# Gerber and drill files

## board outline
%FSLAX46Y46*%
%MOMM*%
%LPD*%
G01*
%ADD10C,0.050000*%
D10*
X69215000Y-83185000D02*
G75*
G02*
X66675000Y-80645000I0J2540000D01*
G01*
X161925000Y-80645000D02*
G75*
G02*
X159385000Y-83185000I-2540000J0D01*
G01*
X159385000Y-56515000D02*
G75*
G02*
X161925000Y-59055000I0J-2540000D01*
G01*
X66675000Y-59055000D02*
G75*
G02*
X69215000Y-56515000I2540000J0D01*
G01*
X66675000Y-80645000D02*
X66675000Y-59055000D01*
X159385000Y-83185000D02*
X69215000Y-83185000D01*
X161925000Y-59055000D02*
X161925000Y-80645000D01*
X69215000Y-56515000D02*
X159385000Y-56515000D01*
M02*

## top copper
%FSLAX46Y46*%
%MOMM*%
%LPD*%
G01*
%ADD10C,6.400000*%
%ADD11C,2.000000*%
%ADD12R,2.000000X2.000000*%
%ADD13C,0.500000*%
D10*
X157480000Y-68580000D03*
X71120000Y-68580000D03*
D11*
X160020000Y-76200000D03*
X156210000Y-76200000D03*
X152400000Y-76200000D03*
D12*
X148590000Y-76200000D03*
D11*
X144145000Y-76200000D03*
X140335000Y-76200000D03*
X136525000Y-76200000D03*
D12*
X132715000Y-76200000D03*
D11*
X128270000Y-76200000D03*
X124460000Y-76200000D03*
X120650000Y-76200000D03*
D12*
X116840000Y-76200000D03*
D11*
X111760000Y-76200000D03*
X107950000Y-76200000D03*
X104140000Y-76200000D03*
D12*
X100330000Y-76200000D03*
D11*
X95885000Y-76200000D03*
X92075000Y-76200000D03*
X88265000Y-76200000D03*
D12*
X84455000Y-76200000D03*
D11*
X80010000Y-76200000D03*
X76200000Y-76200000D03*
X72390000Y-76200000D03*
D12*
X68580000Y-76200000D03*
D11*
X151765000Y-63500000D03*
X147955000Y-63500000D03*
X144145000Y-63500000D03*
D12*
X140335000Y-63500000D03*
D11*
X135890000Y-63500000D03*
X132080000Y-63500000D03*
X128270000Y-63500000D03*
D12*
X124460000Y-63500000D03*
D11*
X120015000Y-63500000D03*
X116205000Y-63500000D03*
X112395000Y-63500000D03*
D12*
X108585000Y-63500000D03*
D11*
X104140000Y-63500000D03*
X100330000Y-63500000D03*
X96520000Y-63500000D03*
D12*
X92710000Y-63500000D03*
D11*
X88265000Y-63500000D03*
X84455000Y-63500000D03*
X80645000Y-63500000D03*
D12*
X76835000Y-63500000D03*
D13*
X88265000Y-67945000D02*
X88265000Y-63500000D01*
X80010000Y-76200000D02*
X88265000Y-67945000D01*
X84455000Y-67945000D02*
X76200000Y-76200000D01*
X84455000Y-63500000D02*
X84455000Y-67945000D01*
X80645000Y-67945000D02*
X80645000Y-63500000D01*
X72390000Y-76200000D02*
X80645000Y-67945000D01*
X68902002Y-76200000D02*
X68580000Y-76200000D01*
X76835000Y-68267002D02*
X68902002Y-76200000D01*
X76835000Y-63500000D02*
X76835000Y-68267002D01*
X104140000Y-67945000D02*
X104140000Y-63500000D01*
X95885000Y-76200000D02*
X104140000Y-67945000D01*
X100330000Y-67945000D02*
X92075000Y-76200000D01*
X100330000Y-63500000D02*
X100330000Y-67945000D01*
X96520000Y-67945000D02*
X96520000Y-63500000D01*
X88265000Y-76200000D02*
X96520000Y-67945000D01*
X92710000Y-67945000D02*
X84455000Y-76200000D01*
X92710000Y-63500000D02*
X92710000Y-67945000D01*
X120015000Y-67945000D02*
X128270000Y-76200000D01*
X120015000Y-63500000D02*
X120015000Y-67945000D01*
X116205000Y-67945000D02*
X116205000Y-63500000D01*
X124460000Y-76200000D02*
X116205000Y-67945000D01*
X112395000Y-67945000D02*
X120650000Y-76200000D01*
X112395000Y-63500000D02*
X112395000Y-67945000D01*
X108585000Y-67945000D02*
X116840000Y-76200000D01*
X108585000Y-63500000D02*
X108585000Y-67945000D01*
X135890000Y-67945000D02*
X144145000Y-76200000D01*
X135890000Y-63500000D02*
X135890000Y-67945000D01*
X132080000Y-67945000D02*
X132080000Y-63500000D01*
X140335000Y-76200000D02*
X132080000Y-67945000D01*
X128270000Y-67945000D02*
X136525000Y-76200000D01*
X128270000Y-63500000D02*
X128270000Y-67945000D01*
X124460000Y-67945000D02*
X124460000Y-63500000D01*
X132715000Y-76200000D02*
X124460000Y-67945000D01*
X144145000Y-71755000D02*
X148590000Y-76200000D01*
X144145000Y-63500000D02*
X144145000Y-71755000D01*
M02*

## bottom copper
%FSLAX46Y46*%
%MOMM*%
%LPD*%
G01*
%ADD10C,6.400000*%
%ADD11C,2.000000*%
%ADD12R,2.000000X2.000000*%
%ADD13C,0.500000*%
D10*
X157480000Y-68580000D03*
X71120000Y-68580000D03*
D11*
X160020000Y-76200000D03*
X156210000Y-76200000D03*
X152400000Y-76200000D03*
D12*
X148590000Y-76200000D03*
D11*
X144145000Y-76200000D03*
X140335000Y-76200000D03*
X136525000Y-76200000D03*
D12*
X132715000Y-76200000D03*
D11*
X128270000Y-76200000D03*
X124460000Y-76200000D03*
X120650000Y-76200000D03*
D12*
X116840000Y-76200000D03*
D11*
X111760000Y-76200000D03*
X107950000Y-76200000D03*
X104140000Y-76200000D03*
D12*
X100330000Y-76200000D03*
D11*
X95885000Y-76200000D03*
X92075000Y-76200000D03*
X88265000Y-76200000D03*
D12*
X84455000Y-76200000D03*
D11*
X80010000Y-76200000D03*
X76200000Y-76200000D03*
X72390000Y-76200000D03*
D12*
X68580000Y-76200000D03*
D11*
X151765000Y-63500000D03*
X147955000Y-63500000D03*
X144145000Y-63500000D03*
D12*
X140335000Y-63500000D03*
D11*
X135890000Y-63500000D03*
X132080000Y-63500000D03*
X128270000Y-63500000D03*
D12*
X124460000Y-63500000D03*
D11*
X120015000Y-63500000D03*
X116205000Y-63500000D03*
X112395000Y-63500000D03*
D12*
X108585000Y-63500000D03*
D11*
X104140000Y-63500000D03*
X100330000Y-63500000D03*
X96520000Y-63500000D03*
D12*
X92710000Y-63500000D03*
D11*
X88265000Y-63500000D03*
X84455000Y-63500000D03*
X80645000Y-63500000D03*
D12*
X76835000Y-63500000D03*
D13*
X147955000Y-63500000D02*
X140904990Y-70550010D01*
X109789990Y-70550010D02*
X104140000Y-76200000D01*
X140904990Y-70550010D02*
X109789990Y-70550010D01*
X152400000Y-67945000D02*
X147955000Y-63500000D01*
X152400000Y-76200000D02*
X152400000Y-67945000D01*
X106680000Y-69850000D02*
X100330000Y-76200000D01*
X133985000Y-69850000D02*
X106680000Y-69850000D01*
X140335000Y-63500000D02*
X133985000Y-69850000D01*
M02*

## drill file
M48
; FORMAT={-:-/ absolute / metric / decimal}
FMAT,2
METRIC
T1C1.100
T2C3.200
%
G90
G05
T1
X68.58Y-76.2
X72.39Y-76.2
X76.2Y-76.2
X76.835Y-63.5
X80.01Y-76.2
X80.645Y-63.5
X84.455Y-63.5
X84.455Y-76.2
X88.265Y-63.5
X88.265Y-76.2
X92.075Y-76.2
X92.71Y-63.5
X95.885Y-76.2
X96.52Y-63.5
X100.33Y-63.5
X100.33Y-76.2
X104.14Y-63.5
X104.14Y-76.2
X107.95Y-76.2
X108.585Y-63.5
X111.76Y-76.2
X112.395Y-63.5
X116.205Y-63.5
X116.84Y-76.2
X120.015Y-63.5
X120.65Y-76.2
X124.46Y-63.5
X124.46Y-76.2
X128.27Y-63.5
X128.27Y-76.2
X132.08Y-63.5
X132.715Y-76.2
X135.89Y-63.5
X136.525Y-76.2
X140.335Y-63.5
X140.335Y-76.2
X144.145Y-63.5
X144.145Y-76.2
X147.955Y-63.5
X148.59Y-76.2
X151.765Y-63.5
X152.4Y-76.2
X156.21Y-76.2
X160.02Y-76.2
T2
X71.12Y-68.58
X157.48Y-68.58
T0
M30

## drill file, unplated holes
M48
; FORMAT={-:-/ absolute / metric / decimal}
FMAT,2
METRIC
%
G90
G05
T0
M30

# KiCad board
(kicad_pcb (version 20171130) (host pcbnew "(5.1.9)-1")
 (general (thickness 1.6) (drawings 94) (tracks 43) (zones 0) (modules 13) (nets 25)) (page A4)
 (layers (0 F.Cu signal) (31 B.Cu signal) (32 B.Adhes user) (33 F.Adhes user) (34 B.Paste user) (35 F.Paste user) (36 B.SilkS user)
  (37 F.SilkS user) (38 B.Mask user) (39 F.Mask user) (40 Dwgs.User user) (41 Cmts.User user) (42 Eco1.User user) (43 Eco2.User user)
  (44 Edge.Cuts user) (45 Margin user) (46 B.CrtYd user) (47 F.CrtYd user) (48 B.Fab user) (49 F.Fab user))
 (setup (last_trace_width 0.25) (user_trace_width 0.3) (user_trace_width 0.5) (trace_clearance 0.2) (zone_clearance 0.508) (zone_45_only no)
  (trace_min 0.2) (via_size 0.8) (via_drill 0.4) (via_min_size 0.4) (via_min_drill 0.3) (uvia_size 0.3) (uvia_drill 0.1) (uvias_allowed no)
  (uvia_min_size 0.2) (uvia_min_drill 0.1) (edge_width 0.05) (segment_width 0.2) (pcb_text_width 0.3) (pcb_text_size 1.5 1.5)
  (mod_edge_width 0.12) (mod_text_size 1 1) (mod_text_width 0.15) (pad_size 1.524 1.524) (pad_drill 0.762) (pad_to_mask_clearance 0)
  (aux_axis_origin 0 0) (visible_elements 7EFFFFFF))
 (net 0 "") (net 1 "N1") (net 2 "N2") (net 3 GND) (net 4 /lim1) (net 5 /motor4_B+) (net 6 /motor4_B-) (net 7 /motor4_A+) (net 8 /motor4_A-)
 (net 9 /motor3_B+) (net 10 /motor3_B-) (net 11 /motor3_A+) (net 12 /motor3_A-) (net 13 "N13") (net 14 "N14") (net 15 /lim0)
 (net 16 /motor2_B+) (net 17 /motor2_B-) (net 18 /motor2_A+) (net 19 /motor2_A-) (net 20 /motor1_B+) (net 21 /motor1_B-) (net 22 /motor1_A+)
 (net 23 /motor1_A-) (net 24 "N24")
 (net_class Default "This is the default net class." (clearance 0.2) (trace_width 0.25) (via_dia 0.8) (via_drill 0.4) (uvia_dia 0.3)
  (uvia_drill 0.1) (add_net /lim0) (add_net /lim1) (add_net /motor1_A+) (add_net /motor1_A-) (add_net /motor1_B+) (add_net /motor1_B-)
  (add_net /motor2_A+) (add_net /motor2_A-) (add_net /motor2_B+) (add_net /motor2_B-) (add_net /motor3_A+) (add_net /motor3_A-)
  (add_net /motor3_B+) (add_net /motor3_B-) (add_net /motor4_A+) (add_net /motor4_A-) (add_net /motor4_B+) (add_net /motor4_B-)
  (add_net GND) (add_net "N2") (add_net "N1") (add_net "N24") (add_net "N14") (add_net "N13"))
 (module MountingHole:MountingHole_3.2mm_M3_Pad (layer F.Cu) (at 157.48 68.58)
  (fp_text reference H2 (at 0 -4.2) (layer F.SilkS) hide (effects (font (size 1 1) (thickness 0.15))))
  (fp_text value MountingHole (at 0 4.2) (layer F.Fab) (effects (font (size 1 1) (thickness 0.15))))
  (pad 1 thru_hole circle (at 0 0) (size 6.4 6.4) (drill 3.2) (layers *.Cu *.Mask)))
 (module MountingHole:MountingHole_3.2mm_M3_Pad (layer F.Cu) (at 71.12 68.58)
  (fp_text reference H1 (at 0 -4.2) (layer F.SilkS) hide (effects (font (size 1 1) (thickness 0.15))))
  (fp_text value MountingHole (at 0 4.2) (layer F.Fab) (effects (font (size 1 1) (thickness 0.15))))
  (pad 1 thru_hole circle (at 0 0) (size 6.4 6.4) (drill 3.2) (layers *.Cu *.Mask)))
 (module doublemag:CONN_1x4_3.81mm (layer F.Cu) (at 148.59 76.2)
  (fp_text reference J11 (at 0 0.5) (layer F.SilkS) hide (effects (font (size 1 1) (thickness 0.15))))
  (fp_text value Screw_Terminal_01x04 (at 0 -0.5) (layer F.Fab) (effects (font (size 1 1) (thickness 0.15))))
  (pad 4 thru_hole circle (at 11.43 0 90) (size 2 2) (drill 1.1) (layers *.Cu *.Mask) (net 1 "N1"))
  (pad 3 thru_hole circle (at 7.62 0 90) (size 2 2) (drill 1.1) (layers *.Cu *.Mask) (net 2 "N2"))
  (pad 2 thru_hole circle (at 3.81 0 90) (size 2 2) (drill 1.1) (layers *.Cu *.Mask) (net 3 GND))
  (pad 1 thru_hole rect (at 0 0 90) (size 2 2) (drill 1.1) (layers *.Cu *.Mask) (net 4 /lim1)))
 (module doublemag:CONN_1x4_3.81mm (layer F.Cu) (at 132.715 76.2)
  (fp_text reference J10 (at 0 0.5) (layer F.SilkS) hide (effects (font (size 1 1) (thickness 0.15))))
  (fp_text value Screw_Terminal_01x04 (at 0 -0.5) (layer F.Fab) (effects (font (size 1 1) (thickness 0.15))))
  (pad 4 thru_hole circle (at 11.43 0 90) (size 2 2) (drill 1.1) (layers *.Cu *.Mask) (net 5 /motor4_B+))
  (pad 3 thru_hole circle (at 7.62 0 90) (size 2 2) (drill 1.1) (layers *.Cu *.Mask) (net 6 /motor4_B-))
  (pad 2 thru_hole circle (at 3.81 0 90) (size 2 2) (drill 1.1) (layers *.Cu *.Mask) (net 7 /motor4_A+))
  (pad 1 thru_hole rect (at 0 0 90) (size 2 2) (drill 1.1) (layers *.Cu *.Mask) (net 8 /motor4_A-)))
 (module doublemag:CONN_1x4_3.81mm (layer F.Cu) (at 116.84 76.2)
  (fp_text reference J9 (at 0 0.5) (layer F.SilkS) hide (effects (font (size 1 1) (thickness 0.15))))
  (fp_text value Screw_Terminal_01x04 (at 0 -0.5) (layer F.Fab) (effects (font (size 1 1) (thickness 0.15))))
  (pad 4 thru_hole circle (at 11.43 0 90) (size 2 2) (drill 1.1) (layers *.Cu *.Mask) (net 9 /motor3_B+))
  (pad 3 thru_hole circle (at 7.62 0 90) (size 2 2) (drill 1.1) (layers *.Cu *.Mask) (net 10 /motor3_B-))
  (pad 2 thru_hole circle (at 3.81 0 90) (size 2 2) (drill 1.1) (layers *.Cu *.Mask) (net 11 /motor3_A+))
  (pad 1 thru_hole rect (at 0 0 90) (size 2 2) (drill 1.1) (layers *.Cu *.Mask) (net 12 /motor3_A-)))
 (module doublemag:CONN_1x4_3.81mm (layer F.Cu) (at 100.33 76.2)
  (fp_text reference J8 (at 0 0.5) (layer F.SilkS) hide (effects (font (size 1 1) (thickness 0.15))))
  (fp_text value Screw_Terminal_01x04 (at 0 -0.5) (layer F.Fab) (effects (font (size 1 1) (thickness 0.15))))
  (pad 4 thru_hole circle (at 11.43 0 90) (size 2 2) (drill 1.1) (layers *.Cu *.Mask) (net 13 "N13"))
  (pad 3 thru_hole circle (at 7.62 0 90) (size 2 2) (drill 1.1) (layers *.Cu *.Mask) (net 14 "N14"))
  (pad 2 thru_hole circle (at 3.81 0 90) (size 2 2) (drill 1.1) (layers *.Cu *.Mask) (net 3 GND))
  (pad 1 thru_hole rect (at 0 0 90) (size 2 2) (drill 1.1) (layers *.Cu *.Mask) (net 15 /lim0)))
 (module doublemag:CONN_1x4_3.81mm (layer F.Cu) (at 84.455 76.2)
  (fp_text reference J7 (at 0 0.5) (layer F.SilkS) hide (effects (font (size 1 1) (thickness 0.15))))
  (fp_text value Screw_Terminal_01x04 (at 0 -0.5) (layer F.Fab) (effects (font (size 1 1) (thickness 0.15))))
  (pad 4 thru_hole circle (at 11.43 0 90) (size 2 2) (drill 1.1) (layers *.Cu *.Mask) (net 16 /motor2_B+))
  (pad 3 thru_hole circle (at 7.62 0 90) (size 2 2) (drill 1.1) (layers *.Cu *.Mask) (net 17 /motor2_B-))
  (pad 2 thru_hole circle (at 3.81 0 90) (size 2 2) (drill 1.1) (layers *.Cu *.Mask) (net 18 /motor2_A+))
  (pad 1 thru_hole rect (at 0 0 90) (size 2 2) (drill 1.1) (layers *.Cu *.Mask) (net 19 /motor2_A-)))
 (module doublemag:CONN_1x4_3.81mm (layer F.Cu) (at 68.58 76.2)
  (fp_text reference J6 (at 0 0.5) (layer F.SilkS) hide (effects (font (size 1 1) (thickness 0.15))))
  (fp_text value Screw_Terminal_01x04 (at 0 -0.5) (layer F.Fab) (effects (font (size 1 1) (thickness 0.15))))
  (pad 4 thru_hole circle (at 11.43 0 90) (size 2 2) (drill 1.1) (layers *.Cu *.Mask) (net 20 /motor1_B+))
  (pad 3 thru_hole circle (at 7.62 0 90) (size 2 2) (drill 1.1) (layers *.Cu *.Mask) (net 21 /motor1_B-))
  (pad 2 thru_hole circle (at 3.81 0 90) (size 2 2) (drill 1.1) (layers *.Cu *.Mask) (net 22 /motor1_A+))
  (pad 1 thru_hole rect (at 0 0 90) (size 2 2) (drill 1.1) (layers *.Cu *.Mask) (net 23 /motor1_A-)))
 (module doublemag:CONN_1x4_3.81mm (layer F.Cu) (at 140.335 63.5)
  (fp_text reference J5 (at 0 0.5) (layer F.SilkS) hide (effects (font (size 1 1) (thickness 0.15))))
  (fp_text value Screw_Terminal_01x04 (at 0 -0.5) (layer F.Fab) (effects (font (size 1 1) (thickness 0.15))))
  (pad 4 thru_hole circle (at 11.43 0 90) (size 2 2) (drill 1.1) (layers *.Cu *.Mask) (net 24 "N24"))
  (pad 3 thru_hole circle (at 7.62 0 90) (size 2 2) (drill 1.1) (layers *.Cu *.Mask) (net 3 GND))
  (pad 2 thru_hole circle (at 3.81 0 90) (size 2 2) (drill 1.1) (layers *.Cu *.Mask) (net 4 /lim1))
  (pad 1 thru_hole rect (at 0 0 90) (size 2 2) (drill 1.1) (layers *.Cu *.Mask) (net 15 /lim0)))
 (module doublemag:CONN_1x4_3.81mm (layer F.Cu) (at 124.46 63.5)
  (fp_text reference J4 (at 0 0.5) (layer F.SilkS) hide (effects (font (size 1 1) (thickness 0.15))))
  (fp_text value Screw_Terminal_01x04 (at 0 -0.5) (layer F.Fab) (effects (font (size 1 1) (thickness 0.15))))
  (pad 4 thru_hole circle (at 11.43 0 90) (size 2 2) (drill 1.1) (layers *.Cu *.Mask) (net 5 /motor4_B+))
  (pad 3 thru_hole circle (at 7.62 0 90) (size 2 2) (drill 1.1) (layers *.Cu *.Mask) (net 6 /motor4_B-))
  (pad 2 thru_hole circle (at 3.81 0 90) (size 2 2) (drill 1.1) (layers *.Cu *.Mask) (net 7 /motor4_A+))
  (pad 1 thru_hole rect (at 0 0 90) (size 2 2) (drill 1.1) (layers *.Cu *.Mask) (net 8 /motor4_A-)))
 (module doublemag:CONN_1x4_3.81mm (layer F.Cu) (at 108.585 63.5)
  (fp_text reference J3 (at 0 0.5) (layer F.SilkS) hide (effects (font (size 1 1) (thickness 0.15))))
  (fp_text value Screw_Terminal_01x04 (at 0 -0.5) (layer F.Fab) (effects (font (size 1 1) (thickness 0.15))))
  (pad 4 thru_hole circle (at 11.43 0 90) (size 2 2) (drill 1.1) (layers *.Cu *.Mask) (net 9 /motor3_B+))
  (pad 3 thru_hole circle (at 7.62 0 90) (size 2 2) (drill 1.1) (layers *.Cu *.Mask) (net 10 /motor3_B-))
  (pad 2 thru_hole circle (at 3.81 0 90) (size 2 2) (drill 1.1) (layers *.Cu *.Mask) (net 11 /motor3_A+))
  (pad 1 thru_hole rect (at 0 0 90) (size 2 2) (drill 1.1) (layers *.Cu *.Mask) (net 12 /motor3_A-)))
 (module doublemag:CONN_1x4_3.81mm (layer F.Cu) (at 92.71 63.5)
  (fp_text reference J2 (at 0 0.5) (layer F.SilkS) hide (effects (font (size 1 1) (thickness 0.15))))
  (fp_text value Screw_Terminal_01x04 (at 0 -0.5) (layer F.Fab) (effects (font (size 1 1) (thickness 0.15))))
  (pad 4 thru_hole circle (at 11.43 0 90) (size 2 2) (drill 1.1) (layers *.Cu *.Mask) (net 16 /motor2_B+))
  (pad 3 thru_hole circle (at 7.62 0 90) (size 2 2) (drill 1.1) (layers *.Cu *.Mask) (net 17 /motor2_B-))
  (pad 2 thru_hole circle (at 3.81 0 90) (size 2 2) (drill 1.1) (layers *.Cu *.Mask) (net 18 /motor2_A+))
  (pad 1 thru_hole rect (at 0 0 90) (size 2 2) (drill 1.1) (layers *.Cu *.Mask) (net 19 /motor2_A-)))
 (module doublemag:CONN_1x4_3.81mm (layer F.Cu) (at 76.835 63.5)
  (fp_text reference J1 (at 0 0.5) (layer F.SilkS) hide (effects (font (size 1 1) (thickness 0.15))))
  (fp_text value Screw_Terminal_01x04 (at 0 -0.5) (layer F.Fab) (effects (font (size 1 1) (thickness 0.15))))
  (pad 4 thru_hole circle (at 11.43 0 90) (size 2 2) (drill 1.1) (layers *.Cu *.Mask) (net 20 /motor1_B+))
  (pad 3 thru_hole circle (at 7.62 0 90) (size 2 2) (drill 1.1) (layers *.Cu *.Mask) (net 21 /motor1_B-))
  (pad 2 thru_hole circle (at 3.81 0 90) (size 2 2) (drill 1.1) (layers *.Cu *.Mask) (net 22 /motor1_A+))
  (pad 1 thru_hole rect (at 0 0 90) (size 2 2) (drill 1.1) (layers *.Cu *.Mask) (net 23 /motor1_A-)))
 (gr_arc (start 69.215 80.645) (end 66.675 80.645) (angle -90) (layer Edge.Cuts) (width 0.05))
 (gr_arc (start 159.385 80.645) (end 159.385 83.185) (angle -90) (layer Edge.Cuts) (width 0.05))
 (gr_arc (start 159.385 59.055) (end 161.925 59.055) (angle -90) (layer Edge.Cuts) (width 0.05))
 (gr_arc (start 69.215 59.055) (end 69.215 56.515) (angle -90) (layer Edge.Cuts) (width 0.05))
 (gr_line (start 66.675 80.645) (end 66.675 59.055) (layer Edge.Cuts) (width 0.05))
 (gr_line (start 159.385 83.185) (end 69.215 83.185) (layer Edge.Cuts) (width 0.05))
 (gr_line (start 161.925 59.055) (end 161.925 80.645) (layer Edge.Cuts) (width 0.05))
 (gr_line (start 69.215 56.515) (end 159.385 56.515) (layer Edge.Cuts) (width 0.05))
 (segment (start 88.265 67.945) (end 88.265 63.5) (width 0.5) (layer F.Cu) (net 20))
 (segment (start 80.01 76.2) (end 88.265 67.945) (width 0.5) (layer F.Cu) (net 20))
 (segment (start 84.455 67.945) (end 76.2 76.2) (width 0.5) (layer F.Cu) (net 21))
 (segment (start 84.455 63.5) (end 84.455 67.945) (width 0.5) (layer F.Cu) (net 21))
 (segment (start 80.645 67.945) (end 80.645 63.5) (width 0.5) (layer F.Cu) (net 22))
 (segment (start 72.39 76.2) (end 80.645 67.945) (width 0.5) (layer F.Cu) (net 22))
 (segment (start 68.902002 76.2) (end 68.58 76.2) (width 0.5) (layer F.Cu) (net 23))
 (segment (start 76.835 68.267002) (end 68.902002 76.2) (width 0.5) (layer F.Cu) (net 23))
 (segment (start 76.835 63.5) (end 76.835 68.267002) (width 0.5) (layer F.Cu) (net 23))
 (segment (start 104.14 67.945) (end 104.14 63.5) (width 0.5) (layer F.Cu) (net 16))
 (segment (start 95.885 76.2) (end 104.14 67.945) (width 0.5) (layer F.Cu) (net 16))
 (segment (start 100.33 67.945) (end 92.075 76.2) (width 0.5) (layer F.Cu) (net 17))
 (segment (start 100.33 63.5) (end 100.33 67.945) (width 0.5) (layer F.Cu) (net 17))
 (segment (start 96.52 67.945) (end 96.52 63.5) (width 0.5) (layer F.Cu) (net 18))
 (segment (start 88.265 76.2) (end 96.52 67.945) (width 0.5) (layer F.Cu) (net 18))
 (segment (start 92.71 67.945) (end 84.455 76.2) (width 0.5) (layer F.Cu) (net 19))
 (segment (start 92.71 63.5) (end 92.71 67.945) (width 0.5) (layer F.Cu) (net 19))
 (segment (start 120.015 67.945) (end 128.27 76.2) (width 0.5) (layer F.Cu) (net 9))
 (segment (start 120.015 63.5) (end 120.015 67.945) (width 0.5) (layer F.Cu) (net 9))
 (segment (start 116.205 67.945) (end 116.205 63.5) (width 0.5) (layer F.Cu) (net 10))
 (segment (start 124.46 76.2) (end 116.205 67.945) (width 0.5) (layer F.Cu) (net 10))
 (segment (start 112.395 67.945) (end 120.65 76.2) (width 0.5) (layer F.Cu) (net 11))
 (segment (start 112.395 63.5) (end 112.395 67.945) (width 0.5) (layer F.Cu) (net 11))
 (segment (start 108.585 67.945) (end 116.84 76.2) (width 0.5) (layer F.Cu) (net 12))
 (segment (start 108.585 63.5) (end 108.585 67.945) (width 0.5) (layer F.Cu) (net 12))
 (segment (start 135.89 67.945) (end 144.145 76.2) (width 0.5) (layer F.Cu) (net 5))
 (segment (start 135.89 63.5) (end 135.89 67.945) (width 0.5) (layer F.Cu) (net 5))
 (segment (start 132.08 67.945) (end 132.08 63.5) (width 0.5) (layer F.Cu) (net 6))
 (segment (start 140.335 76.2) (end 132.08 67.945) (width 0.5) (layer F.Cu) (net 6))
 (segment (start 128.27 67.945) (end 136.525 76.2) (width 0.5) (layer F.Cu) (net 7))
 (segment (start 128.27 63.5) (end 128.27 67.945) (width 0.5) (layer F.Cu) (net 7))
 (segment (start 124.46 67.945) (end 124.46 63.5) (width 0.5) (layer F.Cu) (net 8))
 (segment (start 132.715 76.2) (end 124.46 67.945) (width 0.5) (layer F.Cu) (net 8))
 (segment (start 147.955 63.5) (end 140.90499 70.55001) (width 0.5) (layer B.Cu) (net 3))
 (segment (start 109.78999 70.55001) (end 104.14 76.2) (width 0.5) (layer B.Cu) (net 3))
 (segment (start 140.90499 70.55001) (end 109.78999 70.55001) (width 0.5) (layer B.Cu) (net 3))
 (segment (start 152.4 67.945) (end 147.955 63.5) (width 0.5) (layer B.Cu) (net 3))
 (segment (start 152.4 76.2) (end 152.4 67.945) (width 0.5) (layer B.Cu) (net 3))
 (segment (start 144.145 71.755) (end 148.59 76.2) (width 0.5) (layer F.Cu) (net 4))
 (segment (start 144.145 63.5) (end 144.145 71.755) (width 0.5) (layer F.Cu) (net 4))
 (segment (start 106.68 69.85) (end 100.33 76.2) (width 0.5) (layer B.Cu) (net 15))
 (segment (start 133.985 69.85) (end 106.68 69.85) (width 0.5) (layer B.Cu) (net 15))
 (segment (start 140.335 63.5) (end 133.985 69.85) (width 0.5) (layer B.Cu) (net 15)))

